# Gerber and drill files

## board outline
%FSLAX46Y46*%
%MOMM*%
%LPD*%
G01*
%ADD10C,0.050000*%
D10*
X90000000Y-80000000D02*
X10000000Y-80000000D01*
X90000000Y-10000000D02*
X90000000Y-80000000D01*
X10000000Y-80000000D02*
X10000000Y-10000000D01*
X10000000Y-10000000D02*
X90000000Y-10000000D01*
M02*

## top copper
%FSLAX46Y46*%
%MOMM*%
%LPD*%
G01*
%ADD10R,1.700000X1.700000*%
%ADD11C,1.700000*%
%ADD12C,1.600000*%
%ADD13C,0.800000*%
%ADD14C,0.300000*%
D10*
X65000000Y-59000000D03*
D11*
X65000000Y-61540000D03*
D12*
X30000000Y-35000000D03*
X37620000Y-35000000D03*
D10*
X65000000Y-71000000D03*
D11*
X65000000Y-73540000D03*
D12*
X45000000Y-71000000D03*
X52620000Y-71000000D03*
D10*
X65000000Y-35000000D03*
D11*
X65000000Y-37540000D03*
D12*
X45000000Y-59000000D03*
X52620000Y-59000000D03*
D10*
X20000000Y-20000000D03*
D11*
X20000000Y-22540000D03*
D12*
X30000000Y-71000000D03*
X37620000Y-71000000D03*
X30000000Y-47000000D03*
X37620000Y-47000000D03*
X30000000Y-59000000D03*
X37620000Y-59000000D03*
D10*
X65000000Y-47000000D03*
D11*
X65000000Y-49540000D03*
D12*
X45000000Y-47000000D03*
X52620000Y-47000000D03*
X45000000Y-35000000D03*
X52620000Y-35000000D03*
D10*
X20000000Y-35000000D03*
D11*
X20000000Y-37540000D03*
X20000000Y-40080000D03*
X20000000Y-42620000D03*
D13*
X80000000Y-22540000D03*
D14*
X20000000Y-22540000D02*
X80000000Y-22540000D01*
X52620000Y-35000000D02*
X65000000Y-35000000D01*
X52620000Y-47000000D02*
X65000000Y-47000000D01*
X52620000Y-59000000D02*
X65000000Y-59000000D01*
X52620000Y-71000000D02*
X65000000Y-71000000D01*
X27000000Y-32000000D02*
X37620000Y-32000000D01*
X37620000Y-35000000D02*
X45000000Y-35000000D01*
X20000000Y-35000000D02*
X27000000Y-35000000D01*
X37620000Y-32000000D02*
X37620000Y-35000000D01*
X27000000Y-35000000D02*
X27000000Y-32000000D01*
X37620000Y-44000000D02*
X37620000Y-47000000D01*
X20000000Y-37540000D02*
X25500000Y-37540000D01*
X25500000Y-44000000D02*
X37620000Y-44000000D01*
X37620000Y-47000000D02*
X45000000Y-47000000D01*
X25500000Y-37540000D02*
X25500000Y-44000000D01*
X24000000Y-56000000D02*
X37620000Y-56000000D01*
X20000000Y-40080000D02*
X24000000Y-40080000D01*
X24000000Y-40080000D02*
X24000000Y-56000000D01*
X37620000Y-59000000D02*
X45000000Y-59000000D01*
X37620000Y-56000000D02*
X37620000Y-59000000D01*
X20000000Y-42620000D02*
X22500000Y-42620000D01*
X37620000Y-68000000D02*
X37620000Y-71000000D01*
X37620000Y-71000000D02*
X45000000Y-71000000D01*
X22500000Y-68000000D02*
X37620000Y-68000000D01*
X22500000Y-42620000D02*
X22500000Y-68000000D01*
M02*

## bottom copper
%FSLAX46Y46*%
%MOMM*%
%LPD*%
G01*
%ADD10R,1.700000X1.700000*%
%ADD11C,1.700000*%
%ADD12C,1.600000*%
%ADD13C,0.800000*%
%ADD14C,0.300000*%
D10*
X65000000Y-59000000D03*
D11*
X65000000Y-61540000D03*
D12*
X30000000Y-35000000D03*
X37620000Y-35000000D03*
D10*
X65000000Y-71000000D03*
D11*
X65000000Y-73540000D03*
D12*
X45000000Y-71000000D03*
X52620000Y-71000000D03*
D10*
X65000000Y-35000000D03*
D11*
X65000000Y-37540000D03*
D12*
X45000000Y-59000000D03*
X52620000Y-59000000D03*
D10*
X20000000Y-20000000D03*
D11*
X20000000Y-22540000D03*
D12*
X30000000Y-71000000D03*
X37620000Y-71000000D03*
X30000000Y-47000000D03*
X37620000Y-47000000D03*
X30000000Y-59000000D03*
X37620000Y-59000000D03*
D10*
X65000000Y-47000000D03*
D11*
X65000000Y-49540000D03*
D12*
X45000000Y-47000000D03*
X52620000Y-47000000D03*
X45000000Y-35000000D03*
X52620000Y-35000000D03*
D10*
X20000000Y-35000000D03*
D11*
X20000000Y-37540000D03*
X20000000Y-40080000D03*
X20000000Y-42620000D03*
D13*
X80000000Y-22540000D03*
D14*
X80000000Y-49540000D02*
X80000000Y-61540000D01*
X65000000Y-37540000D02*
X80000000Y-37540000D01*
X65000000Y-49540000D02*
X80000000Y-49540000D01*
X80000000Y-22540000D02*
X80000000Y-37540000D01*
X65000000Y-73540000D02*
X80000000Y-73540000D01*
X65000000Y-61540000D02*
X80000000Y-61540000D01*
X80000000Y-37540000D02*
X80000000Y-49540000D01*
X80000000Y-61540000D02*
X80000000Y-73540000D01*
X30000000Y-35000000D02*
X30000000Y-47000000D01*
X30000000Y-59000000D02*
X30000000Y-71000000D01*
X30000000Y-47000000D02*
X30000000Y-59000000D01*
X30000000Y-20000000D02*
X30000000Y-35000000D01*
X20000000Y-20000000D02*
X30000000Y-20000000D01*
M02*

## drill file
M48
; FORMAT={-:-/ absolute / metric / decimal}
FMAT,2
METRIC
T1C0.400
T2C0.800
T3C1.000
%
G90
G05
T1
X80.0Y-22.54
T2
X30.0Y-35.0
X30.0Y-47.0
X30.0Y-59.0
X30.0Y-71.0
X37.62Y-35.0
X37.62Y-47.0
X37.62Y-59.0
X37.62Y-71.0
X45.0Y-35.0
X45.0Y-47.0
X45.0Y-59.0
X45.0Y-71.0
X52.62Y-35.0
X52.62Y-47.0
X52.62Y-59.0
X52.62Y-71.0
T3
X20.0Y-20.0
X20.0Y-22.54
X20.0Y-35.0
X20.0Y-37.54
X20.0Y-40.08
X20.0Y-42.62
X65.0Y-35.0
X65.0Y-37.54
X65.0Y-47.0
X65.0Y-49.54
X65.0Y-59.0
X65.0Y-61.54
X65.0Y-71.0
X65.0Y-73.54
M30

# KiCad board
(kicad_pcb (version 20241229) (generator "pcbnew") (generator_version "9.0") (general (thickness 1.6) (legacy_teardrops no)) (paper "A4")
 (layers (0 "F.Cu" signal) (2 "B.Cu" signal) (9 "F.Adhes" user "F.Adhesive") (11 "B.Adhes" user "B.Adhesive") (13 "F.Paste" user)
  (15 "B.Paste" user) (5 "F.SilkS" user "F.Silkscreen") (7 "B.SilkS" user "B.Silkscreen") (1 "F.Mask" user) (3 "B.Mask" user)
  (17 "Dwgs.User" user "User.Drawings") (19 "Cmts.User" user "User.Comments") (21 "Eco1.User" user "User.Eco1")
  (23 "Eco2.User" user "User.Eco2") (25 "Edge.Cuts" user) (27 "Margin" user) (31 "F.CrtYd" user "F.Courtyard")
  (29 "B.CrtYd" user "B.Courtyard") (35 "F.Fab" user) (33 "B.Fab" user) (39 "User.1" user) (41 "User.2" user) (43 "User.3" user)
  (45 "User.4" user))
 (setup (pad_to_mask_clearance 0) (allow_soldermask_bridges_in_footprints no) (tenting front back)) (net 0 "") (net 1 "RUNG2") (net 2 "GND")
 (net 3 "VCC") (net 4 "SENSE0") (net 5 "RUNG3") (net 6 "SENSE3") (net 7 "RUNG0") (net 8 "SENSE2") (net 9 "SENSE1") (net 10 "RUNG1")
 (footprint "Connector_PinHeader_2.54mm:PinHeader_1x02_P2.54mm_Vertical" (layer "F.Cu") (at 65 59)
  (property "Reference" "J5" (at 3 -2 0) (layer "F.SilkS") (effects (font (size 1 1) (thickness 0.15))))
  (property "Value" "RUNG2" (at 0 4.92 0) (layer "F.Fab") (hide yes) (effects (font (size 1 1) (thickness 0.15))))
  (pad "1" thru_hole rect (at 0 0) (size 1.7 1.7) (drill 1) (layers "*.Cu" "*.Mask") (remove_unused_layers no) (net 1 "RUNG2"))
  (pad "2" thru_hole circle (at 0 2.54) (size 1.7 1.7) (drill 1) (layers "*.Cu" "*.Mask") (remove_unused_layers no) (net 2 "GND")))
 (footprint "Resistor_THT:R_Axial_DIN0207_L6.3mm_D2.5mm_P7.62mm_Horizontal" (layer "F.Cu") (at 30 35)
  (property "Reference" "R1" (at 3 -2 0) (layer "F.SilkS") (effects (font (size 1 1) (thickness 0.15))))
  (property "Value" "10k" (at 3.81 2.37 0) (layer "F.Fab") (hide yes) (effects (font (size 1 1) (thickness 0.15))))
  (pad "1" thru_hole circle (at 0 0) (size 1.6 1.6) (drill 0.8) (layers "*.Cu" "*.Mask") (remove_unused_layers no) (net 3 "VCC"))
  (pad "2" thru_hole circle (at 7.62 0) (size 1.6 1.6) (drill 0.8) (layers "*.Cu" "*.Mask") (remove_unused_layers no) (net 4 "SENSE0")))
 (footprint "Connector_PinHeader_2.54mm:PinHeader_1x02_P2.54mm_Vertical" (layer "F.Cu") (at 65 71)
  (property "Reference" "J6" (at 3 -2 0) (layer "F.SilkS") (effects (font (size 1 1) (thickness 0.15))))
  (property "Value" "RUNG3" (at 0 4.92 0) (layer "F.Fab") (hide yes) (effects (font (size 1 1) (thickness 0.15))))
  (pad "1" thru_hole rect (at 0 0) (size 1.7 1.7) (drill 1) (layers "*.Cu" "*.Mask") (remove_unused_layers no) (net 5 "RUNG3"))
  (pad "2" thru_hole circle (at 0 2.54) (size 1.7 1.7) (drill 1) (layers "*.Cu" "*.Mask") (remove_unused_layers no) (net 2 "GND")))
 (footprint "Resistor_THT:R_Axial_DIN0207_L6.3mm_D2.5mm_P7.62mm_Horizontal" (layer "F.Cu") (at 45 71)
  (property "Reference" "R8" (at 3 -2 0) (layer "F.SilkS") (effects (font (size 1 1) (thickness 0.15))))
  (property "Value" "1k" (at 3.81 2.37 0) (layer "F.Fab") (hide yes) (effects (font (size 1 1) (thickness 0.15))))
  (pad "1" thru_hole circle (at 0 0) (size 1.6 1.6) (drill 0.8) (layers "*.Cu" "*.Mask") (remove_unused_layers no) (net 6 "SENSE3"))
  (pad "2" thru_hole circle (at 7.62 0) (size 1.6 1.6) (drill 0.8) (layers "*.Cu" "*.Mask") (remove_unused_layers no) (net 5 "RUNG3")))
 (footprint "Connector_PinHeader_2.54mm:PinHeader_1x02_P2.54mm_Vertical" (layer "F.Cu") (at 65 35)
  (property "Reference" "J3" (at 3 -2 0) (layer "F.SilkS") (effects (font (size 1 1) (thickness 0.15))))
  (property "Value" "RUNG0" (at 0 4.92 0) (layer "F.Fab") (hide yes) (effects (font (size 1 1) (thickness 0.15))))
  (pad "1" thru_hole rect (at 0 0) (size 1.7 1.7) (drill 1) (layers "*.Cu" "*.Mask") (remove_unused_layers no) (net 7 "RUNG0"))
  (pad "2" thru_hole circle (at 0 2.54) (size 1.7 1.7) (drill 1) (layers "*.Cu" "*.Mask") (remove_unused_layers no) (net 2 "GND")))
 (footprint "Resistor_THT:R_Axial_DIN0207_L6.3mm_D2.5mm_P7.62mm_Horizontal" (layer "F.Cu") (at 45 59)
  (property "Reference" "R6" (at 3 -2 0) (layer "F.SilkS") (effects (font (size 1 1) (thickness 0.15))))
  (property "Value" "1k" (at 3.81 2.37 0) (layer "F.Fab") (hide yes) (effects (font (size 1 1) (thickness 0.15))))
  (pad "1" thru_hole circle (at 0 0) (size 1.6 1.6) (drill 0.8) (layers "*.Cu" "*.Mask") (remove_unused_layers no) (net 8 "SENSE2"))
  (pad "2" thru_hole circle (at 7.62 0) (size 1.6 1.6) (drill 0.8) (layers "*.Cu" "*.Mask") (remove_unused_layers no) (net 1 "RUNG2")))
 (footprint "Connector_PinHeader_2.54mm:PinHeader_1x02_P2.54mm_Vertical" (layer "F.Cu") (at 20 20)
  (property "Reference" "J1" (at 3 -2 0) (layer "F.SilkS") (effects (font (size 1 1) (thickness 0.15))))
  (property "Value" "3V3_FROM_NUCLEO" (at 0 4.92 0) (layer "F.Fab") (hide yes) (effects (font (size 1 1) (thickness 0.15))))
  (pad "1" thru_hole rect (at 0 0) (size 1.7 1.7) (drill 1) (layers "*.Cu" "*.Mask") (remove_unused_layers no) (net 3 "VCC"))
  (pad "2" thru_hole circle (at 0 2.54) (size 1.7 1.7) (drill 1) (layers "*.Cu" "*.Mask") (remove_unused_layers no) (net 2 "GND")))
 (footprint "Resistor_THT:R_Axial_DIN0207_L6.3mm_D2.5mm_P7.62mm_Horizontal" (layer "F.Cu") (at 30 71)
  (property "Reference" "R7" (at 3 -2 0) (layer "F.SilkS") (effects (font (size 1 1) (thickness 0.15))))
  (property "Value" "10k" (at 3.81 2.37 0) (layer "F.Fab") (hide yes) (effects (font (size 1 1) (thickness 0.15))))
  (pad "1" thru_hole circle (at 0 0) (size 1.6 1.6) (drill 0.8) (layers "*.Cu" "*.Mask") (remove_unused_layers no) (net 3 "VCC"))
  (pad "2" thru_hole circle (at 7.62 0) (size 1.6 1.6) (drill 0.8) (layers "*.Cu" "*.Mask") (remove_unused_layers no) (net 6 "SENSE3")))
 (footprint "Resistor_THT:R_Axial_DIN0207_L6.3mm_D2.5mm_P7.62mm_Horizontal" (layer "F.Cu") (at 30 47)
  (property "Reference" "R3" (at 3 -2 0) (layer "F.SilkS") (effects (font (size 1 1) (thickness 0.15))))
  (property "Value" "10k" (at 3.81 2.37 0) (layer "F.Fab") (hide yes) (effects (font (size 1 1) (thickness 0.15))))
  (pad "1" thru_hole circle (at 0 0) (size 1.6 1.6) (drill 0.8) (layers "*.Cu" "*.Mask") (remove_unused_layers no) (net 3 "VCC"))
  (pad "2" thru_hole circle (at 7.62 0) (size 1.6 1.6) (drill 0.8) (layers "*.Cu" "*.Mask") (remove_unused_layers no) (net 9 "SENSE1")))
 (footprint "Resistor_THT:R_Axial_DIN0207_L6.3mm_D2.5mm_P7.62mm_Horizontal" (layer "F.Cu") (at 30 59)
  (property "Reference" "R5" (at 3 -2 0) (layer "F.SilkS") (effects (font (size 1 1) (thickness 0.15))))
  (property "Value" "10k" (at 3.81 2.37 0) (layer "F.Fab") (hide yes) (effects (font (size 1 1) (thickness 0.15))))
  (pad "1" thru_hole circle (at 0 0) (size 1.6 1.6) (drill 0.8) (layers "*.Cu" "*.Mask") (remove_unused_layers no) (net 3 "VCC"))
  (pad "2" thru_hole circle (at 7.62 0) (size 1.6 1.6) (drill 0.8) (layers "*.Cu" "*.Mask") (remove_unused_layers no) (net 8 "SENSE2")))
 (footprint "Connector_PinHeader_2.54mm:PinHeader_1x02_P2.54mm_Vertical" (layer "F.Cu") (at 65 47)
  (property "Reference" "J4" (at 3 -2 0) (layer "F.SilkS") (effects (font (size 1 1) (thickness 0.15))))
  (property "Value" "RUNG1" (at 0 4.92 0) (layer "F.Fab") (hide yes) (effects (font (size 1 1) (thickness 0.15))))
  (pad "1" thru_hole rect (at 0 0) (size 1.7 1.7) (drill 1) (layers "*.Cu" "*.Mask") (remove_unused_layers no) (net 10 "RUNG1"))
  (pad "2" thru_hole circle (at 0 2.54) (size 1.7 1.7) (drill 1) (layers "*.Cu" "*.Mask") (remove_unused_layers no) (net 2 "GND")))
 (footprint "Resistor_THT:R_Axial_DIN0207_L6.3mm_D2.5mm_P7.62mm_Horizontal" (layer "F.Cu") (at 45 47)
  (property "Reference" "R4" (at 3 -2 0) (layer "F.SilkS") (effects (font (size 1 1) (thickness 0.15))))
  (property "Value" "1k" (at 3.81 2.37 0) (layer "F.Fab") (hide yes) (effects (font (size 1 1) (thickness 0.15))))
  (pad "1" thru_hole circle (at 0 0) (size 1.6 1.6) (drill 0.8) (layers "*.Cu" "*.Mask") (remove_unused_layers no) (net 9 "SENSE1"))
  (pad "2" thru_hole circle (at 7.62 0) (size 1.6 1.6) (drill 0.8) (layers "*.Cu" "*.Mask") (remove_unused_layers no) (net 10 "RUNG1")))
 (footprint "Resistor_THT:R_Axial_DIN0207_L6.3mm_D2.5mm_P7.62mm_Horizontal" (layer "F.Cu") (at 45 35)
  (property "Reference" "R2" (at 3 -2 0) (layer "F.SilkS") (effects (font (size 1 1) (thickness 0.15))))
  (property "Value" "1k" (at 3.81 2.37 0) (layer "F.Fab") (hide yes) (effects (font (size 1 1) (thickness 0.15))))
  (pad "1" thru_hole circle (at 0 0) (size 1.6 1.6) (drill 0.8) (layers "*.Cu" "*.Mask") (remove_unused_layers no) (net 4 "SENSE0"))
  (pad "2" thru_hole circle (at 7.62 0) (size 1.6 1.6) (drill 0.8) (layers "*.Cu" "*.Mask") (remove_unused_layers no) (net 7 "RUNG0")))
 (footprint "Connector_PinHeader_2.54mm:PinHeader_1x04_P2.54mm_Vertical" (layer "F.Cu") (at 20 35)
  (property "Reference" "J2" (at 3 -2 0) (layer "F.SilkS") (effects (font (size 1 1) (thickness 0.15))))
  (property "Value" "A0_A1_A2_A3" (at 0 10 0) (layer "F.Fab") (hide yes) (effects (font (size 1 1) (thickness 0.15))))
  (pad "1" thru_hole rect (at 0 0) (size 1.7 1.7) (drill 1) (layers "*.Cu" "*.Mask") (remove_unused_layers no) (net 4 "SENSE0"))
  (pad "2" thru_hole circle (at 0 2.54) (size 1.7 1.7) (drill 1) (layers "*.Cu" "*.Mask") (remove_unused_layers no) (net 9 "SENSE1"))
  (pad "3" thru_hole circle (at 0 5.08) (size 1.7 1.7) (drill 1) (layers "*.Cu" "*.Mask") (remove_unused_layers no) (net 8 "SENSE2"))
  (pad "4" thru_hole circle (at 0 7.62) (size 1.7 1.7) (drill 1) (layers "*.Cu" "*.Mask") (remove_unused_layers no) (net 6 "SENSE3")))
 (gr_line (start 90 80) (end 10 80) (stroke (width 0.05) (type default)) (layer "Edge.Cuts"))
 (gr_line (start 90 10) (end 90 80) (stroke (width 0.05) (type default)) (layer "Edge.Cuts"))
 (gr_line (start 10 80) (end 10 10) (stroke (width 0.05) (type default)) (layer "Edge.Cuts"))
 (gr_line (start 10 10) (end 90 10) (stroke (width 0.05) (type default)) (layer "Edge.Cuts"))
 (segment (start 20 22.54) (end 80 22.54) (width 0.3) (layer "F.Cu") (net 2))
 (via (at 80 22.54) (size 0.8) (drill 0.4) (layers "F.Cu" "B.Cu") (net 2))
 (segment (start 80 49.54) (end 80 61.54) (width 0.3) (layer "B.Cu") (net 2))
 (segment (start 65 37.54) (end 80 37.54) (width 0.3) (layer "B.Cu") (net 2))
 (segment (start 65 49.54) (end 80 49.54) (width 0.3) (layer "B.Cu") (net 2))
 (segment (start 80 22.54) (end 80 37.54) (width 0.3) (layer "B.Cu") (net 2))
 (segment (start 65 73.54) (end 80 73.54) (width 0.3) (layer "B.Cu") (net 2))
 (segment (start 65 61.54) (end 80 61.54) (width 0.3) (layer "B.Cu") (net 2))
 (segment (start 80 37.54) (end 80 49.54) (width 0.3) (layer "B.Cu") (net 2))
 (segment (start 80 61.54) (end 80 73.54) (width 0.3) (layer "B.Cu") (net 2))
 (segment (start 52.62 35) (end 65 35) (width 0.3) (layer "F.Cu") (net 7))
 (segment (start 52.62 47) (end 65 47) (width 0.3) (layer "F.Cu") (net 10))
 (segment (start 52.62 59) (end 65 59) (width 0.3) (layer "F.Cu") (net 1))
 (segment (start 52.62 71) (end 65 71) (width 0.3) (layer "F.Cu") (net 5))
 (segment (start 27 32) (end 37.62 32) (width 0.3) (layer "F.Cu") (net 4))
 (segment (start 37.62 35) (end 45 35) (width 0.3) (layer "F.Cu") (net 4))
 (segment (start 20 35) (end 27 35) (width 0.3) (layer "F.Cu") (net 4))
 (segment (start 37.62 32) (end 37.62 35) (width 0.3) (layer "F.Cu") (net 4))
 (segment (start 27 35) (end 27 32) (width 0.3) (layer "F.Cu") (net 4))
 (segment (start 37.62 44) (end 37.62 47) (width 0.3) (layer "F.Cu") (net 9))
 (segment (start 20 37.54) (end 25.5 37.54) (width 0.3) (layer "F.Cu") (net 9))
 (segment (start 25.5 44) (end 37.62 44) (width 0.3) (layer "F.Cu") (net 9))
 (segment (start 37.62 47) (end 45 47) (width 0.3) (layer "F.Cu") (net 9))
 (segment (start 25.5 37.54) (end 25.5 44) (width 0.3) (layer "F.Cu") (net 9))
 (segment (start 24 56) (end 37.62 56) (width 0.3) (layer "F.Cu") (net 8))
 (segment (start 20 40.08) (end 24 40.08) (width 0.3) (layer "F.Cu") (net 8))
 (segment (start 24 40.08) (end 24 56) (width 0.3) (layer "F.Cu") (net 8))
 (segment (start 37.62 59) (end 45 59) (width 0.3) (layer "F.Cu") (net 8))
 (segment (start 37.62 56) (end 37.62 59) (width 0.3) (layer "F.Cu") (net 8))
 (segment (start 20 42.62) (end 22.5 42.62) (width 0.3) (layer "F.Cu") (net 6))
 (segment (start 37.62 68) (end 37.62 71) (width 0.3) (layer "F.Cu") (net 6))
 (segment (start 37.62 71) (end 45 71) (width 0.3) (layer "F.Cu") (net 6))
 (segment (start 22.5 68) (end 37.62 68) (width 0.3) (layer "F.Cu") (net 6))
 (segment (start 22.5 42.62) (end 22.5 68) (width 0.3) (layer "F.Cu") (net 6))
 (segment (start 30 35) (end 30 47) (width 0.3) (layer "B.Cu") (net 3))
 (segment (start 30 59) (end 30 71) (width 0.3) (layer "B.Cu") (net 3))
 (segment (start 30 47) (end 30 59) (width 0.3) (layer "B.Cu") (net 3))
 (segment (start 30 20) (end 30 35) (width 0.3) (layer "B.Cu") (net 3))
 (segment (start 20 20) (end 30 20) (width 0.3) (layer "B.Cu") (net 3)))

